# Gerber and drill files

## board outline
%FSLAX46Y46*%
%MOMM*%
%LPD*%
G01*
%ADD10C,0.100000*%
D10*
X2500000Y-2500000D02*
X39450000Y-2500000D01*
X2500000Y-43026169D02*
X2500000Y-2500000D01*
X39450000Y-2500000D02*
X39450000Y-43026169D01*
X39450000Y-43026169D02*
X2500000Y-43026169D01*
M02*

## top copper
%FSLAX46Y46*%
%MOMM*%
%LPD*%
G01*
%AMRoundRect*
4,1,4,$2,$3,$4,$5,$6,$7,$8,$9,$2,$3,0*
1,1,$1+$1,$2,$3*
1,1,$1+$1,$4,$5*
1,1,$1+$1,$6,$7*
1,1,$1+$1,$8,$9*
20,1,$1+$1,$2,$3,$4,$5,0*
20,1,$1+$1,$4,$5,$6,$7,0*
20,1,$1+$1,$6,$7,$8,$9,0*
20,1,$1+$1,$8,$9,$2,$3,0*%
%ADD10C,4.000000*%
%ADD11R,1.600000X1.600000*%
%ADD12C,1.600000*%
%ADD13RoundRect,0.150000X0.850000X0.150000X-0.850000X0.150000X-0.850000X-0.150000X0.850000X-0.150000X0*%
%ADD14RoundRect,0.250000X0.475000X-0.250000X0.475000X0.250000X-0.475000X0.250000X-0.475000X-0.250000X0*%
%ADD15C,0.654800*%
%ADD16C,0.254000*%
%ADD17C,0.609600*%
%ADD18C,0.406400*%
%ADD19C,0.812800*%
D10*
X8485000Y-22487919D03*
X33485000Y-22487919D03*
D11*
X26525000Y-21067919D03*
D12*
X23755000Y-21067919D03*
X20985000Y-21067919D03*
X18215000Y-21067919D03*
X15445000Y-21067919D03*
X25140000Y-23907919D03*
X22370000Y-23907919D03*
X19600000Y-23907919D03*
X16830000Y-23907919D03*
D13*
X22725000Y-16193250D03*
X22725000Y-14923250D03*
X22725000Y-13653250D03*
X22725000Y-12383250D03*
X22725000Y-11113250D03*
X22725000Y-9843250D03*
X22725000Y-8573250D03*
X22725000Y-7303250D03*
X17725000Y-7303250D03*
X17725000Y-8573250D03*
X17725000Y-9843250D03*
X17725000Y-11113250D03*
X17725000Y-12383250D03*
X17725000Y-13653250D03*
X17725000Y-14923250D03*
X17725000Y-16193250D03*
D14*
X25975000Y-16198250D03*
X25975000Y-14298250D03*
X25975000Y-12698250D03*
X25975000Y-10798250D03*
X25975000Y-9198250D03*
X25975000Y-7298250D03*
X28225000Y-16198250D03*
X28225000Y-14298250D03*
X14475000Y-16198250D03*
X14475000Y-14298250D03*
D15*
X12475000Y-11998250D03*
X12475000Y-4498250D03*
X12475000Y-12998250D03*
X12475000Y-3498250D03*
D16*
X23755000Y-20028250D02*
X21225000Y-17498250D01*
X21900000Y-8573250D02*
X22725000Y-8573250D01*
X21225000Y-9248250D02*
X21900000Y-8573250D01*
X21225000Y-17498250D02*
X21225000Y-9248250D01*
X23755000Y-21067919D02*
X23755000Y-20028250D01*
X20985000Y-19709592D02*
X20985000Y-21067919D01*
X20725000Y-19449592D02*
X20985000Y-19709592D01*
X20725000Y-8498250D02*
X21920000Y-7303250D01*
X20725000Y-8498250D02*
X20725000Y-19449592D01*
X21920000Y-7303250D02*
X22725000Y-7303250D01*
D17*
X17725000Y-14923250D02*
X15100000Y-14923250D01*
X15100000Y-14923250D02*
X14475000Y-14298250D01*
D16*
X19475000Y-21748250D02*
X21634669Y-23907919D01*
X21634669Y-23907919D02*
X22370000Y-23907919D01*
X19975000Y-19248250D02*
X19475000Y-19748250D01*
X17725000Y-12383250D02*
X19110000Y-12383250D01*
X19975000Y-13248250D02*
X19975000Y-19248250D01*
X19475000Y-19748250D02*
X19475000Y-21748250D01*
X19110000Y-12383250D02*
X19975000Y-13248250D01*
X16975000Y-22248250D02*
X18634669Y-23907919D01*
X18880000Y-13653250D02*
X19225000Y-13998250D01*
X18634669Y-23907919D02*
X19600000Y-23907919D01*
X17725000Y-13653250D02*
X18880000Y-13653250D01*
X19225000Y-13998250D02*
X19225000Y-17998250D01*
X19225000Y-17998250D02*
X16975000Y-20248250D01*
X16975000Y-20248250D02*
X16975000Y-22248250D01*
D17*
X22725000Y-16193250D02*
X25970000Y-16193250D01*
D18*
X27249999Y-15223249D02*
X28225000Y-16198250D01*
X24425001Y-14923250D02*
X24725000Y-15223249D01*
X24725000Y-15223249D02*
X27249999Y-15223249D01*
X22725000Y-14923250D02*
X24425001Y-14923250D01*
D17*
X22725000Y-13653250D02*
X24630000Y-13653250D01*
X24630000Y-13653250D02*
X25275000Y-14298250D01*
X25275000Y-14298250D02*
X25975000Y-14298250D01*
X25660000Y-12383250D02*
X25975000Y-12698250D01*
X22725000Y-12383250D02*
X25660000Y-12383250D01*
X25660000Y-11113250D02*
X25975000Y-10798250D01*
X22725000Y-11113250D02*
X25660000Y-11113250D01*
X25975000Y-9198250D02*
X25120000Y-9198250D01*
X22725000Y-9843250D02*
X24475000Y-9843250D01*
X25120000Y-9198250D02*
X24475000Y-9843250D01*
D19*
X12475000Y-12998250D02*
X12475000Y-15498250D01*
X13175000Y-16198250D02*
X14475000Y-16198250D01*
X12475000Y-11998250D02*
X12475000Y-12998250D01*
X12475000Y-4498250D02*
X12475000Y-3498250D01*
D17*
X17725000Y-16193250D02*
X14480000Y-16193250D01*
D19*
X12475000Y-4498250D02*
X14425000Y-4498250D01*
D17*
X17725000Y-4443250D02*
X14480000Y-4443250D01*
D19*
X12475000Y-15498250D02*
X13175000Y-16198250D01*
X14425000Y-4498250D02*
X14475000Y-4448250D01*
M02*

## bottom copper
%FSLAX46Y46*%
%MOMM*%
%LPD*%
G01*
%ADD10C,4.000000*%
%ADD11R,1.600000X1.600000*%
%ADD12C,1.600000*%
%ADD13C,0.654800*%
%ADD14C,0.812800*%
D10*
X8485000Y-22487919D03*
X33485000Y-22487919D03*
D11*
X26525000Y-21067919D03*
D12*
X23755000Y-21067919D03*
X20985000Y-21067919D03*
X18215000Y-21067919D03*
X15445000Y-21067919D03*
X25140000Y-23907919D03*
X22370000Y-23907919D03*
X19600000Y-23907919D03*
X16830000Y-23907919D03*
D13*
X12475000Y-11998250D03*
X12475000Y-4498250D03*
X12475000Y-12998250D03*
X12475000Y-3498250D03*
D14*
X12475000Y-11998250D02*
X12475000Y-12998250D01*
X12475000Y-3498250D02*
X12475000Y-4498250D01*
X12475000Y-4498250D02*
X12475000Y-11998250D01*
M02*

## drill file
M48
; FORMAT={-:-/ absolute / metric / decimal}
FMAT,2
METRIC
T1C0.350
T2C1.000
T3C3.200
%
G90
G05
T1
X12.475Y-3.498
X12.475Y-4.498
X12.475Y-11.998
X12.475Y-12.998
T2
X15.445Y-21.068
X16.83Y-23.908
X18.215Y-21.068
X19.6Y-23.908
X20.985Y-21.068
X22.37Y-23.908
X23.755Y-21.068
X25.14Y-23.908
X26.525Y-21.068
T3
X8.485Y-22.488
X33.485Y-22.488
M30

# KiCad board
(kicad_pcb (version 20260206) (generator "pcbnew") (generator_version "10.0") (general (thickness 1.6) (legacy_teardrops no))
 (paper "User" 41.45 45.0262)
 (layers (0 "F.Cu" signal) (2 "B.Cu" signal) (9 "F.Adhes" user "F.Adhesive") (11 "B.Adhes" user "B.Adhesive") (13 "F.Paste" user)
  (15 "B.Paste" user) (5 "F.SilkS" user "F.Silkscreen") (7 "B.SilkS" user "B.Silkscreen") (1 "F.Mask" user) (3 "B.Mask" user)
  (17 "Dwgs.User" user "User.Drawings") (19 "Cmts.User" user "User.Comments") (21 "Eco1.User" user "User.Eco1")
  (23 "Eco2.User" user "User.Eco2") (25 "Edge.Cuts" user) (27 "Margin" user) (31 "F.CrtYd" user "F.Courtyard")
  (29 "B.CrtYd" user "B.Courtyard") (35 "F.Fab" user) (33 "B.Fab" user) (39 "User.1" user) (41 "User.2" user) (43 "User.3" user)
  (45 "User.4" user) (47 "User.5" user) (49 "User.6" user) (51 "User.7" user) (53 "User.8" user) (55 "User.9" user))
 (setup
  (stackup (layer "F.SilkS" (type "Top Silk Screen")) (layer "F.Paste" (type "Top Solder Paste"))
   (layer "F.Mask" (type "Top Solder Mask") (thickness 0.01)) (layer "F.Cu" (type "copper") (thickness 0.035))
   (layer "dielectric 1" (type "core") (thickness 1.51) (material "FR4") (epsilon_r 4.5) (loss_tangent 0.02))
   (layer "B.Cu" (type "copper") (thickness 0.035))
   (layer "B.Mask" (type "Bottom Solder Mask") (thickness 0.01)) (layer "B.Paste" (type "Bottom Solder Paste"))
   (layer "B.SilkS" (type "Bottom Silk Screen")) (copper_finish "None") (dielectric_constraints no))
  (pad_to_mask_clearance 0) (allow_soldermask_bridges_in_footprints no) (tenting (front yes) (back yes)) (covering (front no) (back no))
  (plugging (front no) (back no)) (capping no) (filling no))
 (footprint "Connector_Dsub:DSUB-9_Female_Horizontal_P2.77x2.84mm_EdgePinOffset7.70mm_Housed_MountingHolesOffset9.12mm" (layer "F.Cu")
  (at 26.525 21.067919)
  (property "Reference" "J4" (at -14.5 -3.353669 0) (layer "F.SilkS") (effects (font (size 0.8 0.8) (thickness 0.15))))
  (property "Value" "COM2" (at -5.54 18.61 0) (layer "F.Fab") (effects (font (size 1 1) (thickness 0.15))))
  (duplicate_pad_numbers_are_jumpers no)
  (pad "0" thru_hole circle (at -18.04 1.42) (size 4 4) (drill 3.2) (layers "*.Cu" "*.Mask") (remove_unused_layers no)
   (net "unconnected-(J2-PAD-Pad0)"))
  (pad "0" thru_hole circle (at 6.96 1.42) (size 4 4) (drill 3.2) (layers "*.Cu" "*.Mask") (remove_unused_layers no)
   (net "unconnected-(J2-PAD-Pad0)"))
  (pad "1" thru_hole rect (at 0 0) (size 1.6 1.6) (drill 1) (layers "*.Cu" "*.Mask") (remove_unused_layers no) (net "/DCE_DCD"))
  (pad "2" thru_hole circle (at -2.77 0) (size 1.6 1.6) (drill 1) (layers "*.Cu" "*.Mask") (remove_unused_layers no) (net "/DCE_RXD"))
  (pad "3" thru_hole circle (at -5.54 0) (size 1.6 1.6) (drill 1) (layers "*.Cu" "*.Mask") (remove_unused_layers no) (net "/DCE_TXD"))
  (pad "4" thru_hole circle (at -8.31 0) (size 1.6 1.6) (drill 1) (layers "*.Cu" "*.Mask") (remove_unused_layers no) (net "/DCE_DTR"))
  (pad "5" thru_hole circle (at -11.08 0) (size 1.6 1.6) (drill 1) (layers "*.Cu" "*.Mask") (remove_unused_layers no) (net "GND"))
  (pad "6" thru_hole circle (at -1.385 2.84) (size 1.6 1.6) (drill 1) (layers "*.Cu" "*.Mask") (remove_unused_layers no) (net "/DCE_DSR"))
  (pad "7" thru_hole circle (at -4.155 2.84) (size 1.6 1.6) (drill 1) (layers "*.Cu" "*.Mask") (remove_unused_layers no) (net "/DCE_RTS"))
  (pad "8" thru_hole circle (at -6.925 2.84) (size 1.6 1.6) (drill 1) (layers "*.Cu" "*.Mask") (remove_unused_layers no) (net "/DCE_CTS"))
  (pad "9" thru_hole circle (at -9.695 2.84) (size 1.6 1.6) (drill 1) (layers "*.Cu" "*.Mask") (remove_unused_layers no) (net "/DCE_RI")))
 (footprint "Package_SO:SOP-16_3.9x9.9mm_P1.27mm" (layer "F.Cu") (at 20.225 11.74825 180)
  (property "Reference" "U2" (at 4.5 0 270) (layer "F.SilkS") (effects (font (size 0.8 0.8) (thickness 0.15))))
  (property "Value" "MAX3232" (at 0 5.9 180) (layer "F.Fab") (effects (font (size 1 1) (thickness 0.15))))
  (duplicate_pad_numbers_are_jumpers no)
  (pad "1" smd roundrect (at -2.5 -4.445 180) (size 2 0.6) (layers "F.Cu" "F.Mask" "F.Paste") (roundrect_rratio 0.25) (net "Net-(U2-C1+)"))
  (pad "2" smd roundrect (at -2.5 -3.175 180) (size 2 0.6) (layers "F.Cu" "F.Mask" "F.Paste") (roundrect_rratio 0.25) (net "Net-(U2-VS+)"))
  (pad "3" smd roundrect (at -2.5 -1.905 180) (size 2 0.6) (layers "F.Cu" "F.Mask" "F.Paste") (roundrect_rratio 0.25) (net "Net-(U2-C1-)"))
  (pad "4" smd roundrect (at -2.5 -0.635 180) (size 2 0.6) (layers "F.Cu" "F.Mask" "F.Paste") (roundrect_rratio 0.25) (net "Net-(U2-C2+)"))
  (pad "5" smd roundrect (at -2.5 0.635 180) (size 2 0.6) (layers "F.Cu" "F.Mask" "F.Paste") (roundrect_rratio 0.25) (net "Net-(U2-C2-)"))
  (pad "6" smd roundrect (at -2.5 1.905 180) (size 2 0.6) (layers "F.Cu" "F.Mask" "F.Paste") (roundrect_rratio 0.25) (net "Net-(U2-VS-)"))
  (pad "7" smd roundrect (at -2.5 3.175 180) (size 2 0.6) (layers "F.Cu" "F.Mask" "F.Paste") (roundrect_rratio 0.25) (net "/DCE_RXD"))
  (pad "8" smd roundrect (at -2.5 4.445 180) (size 2 0.6) (layers "F.Cu" "F.Mask" "F.Paste") (roundrect_rratio 0.25) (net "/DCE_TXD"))
  (pad "9" smd roundrect (at 2.5 4.445 180) (size 2 0.6) (layers "F.Cu" "F.Mask" "F.Paste") (roundrect_rratio 0.25) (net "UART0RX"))
  (pad "10" smd roundrect (at 2.5 3.175 180) (size 2 0.6) (layers "F.Cu" "F.Mask" "F.Paste") (roundrect_rratio 0.25) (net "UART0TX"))
  (pad "11" smd roundrect (at 2.5 1.905 180) (size 2 0.6) (layers "F.Cu" "F.Mask" "F.Paste") (roundrect_rratio 0.25) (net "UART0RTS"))
  (pad "12" smd roundrect (at 2.5 0.635 180) (size 2 0.6) (layers "F.Cu" "F.Mask" "F.Paste") (roundrect_rratio 0.25) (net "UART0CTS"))
  (pad "13" smd roundrect (at 2.5 -0.635 180) (size 2 0.6) (layers "F.Cu" "F.Mask" "F.Paste") (roundrect_rratio 0.25) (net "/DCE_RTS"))
  (pad "14" smd roundrect (at 2.5 -1.905 180) (size 2 0.6) (layers "F.Cu" "F.Mask" "F.Paste") (roundrect_rratio 0.25) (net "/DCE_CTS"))
  (pad "15" smd roundrect (at 2.5 -3.175 180) (size 2 0.6) (layers "F.Cu" "F.Mask" "F.Paste") (roundrect_rratio 0.25) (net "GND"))
  (pad "16" smd roundrect (at 2.5 -4.445 180) (size 2 0.6) (layers "F.Cu" "F.Mask" "F.Paste") (roundrect_rratio 0.25) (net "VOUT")))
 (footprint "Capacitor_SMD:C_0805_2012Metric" (layer "F.Cu") (at 25.975 15.24825 90)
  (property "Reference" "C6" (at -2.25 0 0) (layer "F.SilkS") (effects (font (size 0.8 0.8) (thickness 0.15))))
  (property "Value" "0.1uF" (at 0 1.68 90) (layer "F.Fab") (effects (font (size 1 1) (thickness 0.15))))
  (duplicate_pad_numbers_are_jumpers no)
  (pad "1" smd roundrect (at -0.95 0 90) (size 1 1.45) (layers "F.Cu" "F.Mask" "F.Paste") (roundrect_rratio 0.25) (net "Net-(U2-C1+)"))
  (pad "2" smd roundrect (at 0.95 0 90) (size 1 1.45) (layers "F.Cu" "F.Mask" "F.Paste") (roundrect_rratio 0.25) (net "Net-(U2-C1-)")))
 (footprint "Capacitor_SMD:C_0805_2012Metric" (layer "F.Cu") (at 25.975 11.74825 90)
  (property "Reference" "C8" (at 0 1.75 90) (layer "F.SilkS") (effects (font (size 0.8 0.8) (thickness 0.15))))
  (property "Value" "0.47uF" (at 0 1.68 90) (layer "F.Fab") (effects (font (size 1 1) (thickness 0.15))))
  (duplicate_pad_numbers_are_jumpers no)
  (pad "1" smd roundrect (at -0.95 0 90) (size 1 1.45) (layers "F.Cu" "F.Mask" "F.Paste") (roundrect_rratio 0.25) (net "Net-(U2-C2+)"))
  (pad "2" smd roundrect (at 0.95 0 90) (size 1 1.45) (layers "F.Cu" "F.Mask" "F.Paste") (roundrect_rratio 0.25) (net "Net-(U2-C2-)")))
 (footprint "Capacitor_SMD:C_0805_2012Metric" (layer "F.Cu") (at 25.975 8.24825 90)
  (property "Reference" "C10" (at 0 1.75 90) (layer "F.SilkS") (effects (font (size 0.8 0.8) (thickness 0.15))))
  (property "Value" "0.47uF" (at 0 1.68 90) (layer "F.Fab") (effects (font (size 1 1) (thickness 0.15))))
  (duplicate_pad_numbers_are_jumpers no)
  (pad "1" smd roundrect (at -0.95 0 90) (size 1 1.45) (layers "F.Cu" "F.Mask" "F.Paste") (roundrect_rratio 0.25) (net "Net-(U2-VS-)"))
  (pad "2" smd roundrect (at 0.95 0 90) (size 1 1.45) (layers "F.Cu" "F.Mask" "F.Paste") (roundrect_rratio 0.25) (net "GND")))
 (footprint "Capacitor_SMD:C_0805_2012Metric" (layer "F.Cu") (at 28.225 15.24825 90)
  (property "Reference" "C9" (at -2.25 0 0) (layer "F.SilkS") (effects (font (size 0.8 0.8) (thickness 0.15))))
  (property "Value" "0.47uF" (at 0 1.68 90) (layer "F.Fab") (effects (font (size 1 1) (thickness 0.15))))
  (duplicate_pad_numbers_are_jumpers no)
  (pad "1" smd roundrect (at -0.95 0 90) (size 1 1.45) (layers "F.Cu" "F.Mask" "F.Paste") (roundrect_rratio 0.25) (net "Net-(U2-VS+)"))
  (pad "2" smd roundrect (at 0.95 0 90) (size 1 1.45) (layers "F.Cu" "F.Mask" "F.Paste") (roundrect_rratio 0.25) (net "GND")))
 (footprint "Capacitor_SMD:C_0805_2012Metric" (layer "F.Cu") (at 14.475 15.24825 90)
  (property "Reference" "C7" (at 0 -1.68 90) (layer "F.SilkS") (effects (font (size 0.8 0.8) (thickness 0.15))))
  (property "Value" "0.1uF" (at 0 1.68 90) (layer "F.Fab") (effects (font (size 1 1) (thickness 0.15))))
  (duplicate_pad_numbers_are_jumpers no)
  (pad "1" smd roundrect (at -0.95 0 90) (size 1 1.45) (layers "F.Cu" "F.Mask" "F.Paste") (roundrect_rratio 0.25) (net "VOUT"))
  (pad "2" smd roundrect (at 0.95 0 90) (size 1 1.45) (layers "F.Cu" "F.Mask" "F.Paste") (roundrect_rratio 0.25) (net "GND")))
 (gr_line (start 2.5 2.5) (end 39.45 2.5) (stroke (width 0.1) (type default)) (layer "Edge.Cuts"))
 (gr_line (start 2.5 43.026169) (end 2.5 2.5) (stroke (width 0.1) (type default)) (layer "Edge.Cuts"))
 (gr_line (start 39.45 2.5) (end 39.45 43.026169) (stroke (width 0.1) (type default)) (layer "Edge.Cuts"))
 (gr_line (start 39.45 43.026169) (end 2.5 43.026169) (stroke (width 0.1) (type default)) (layer "Edge.Cuts"))
 (segment (start 23.755 20.02825) (end 21.225 17.49825) (width 0.254) (layer "F.Cu") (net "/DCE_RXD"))
 (segment (start 21.9 8.57325) (end 22.725 8.57325) (width 0.254) (layer "F.Cu") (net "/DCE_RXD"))
 (segment (start 21.225 9.24825) (end 21.9 8.57325) (width 0.254) (layer "F.Cu") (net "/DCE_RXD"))
 (segment (start 21.225 17.49825) (end 21.225 9.24825) (width 0.254) (layer "F.Cu") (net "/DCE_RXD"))
 (segment (start 23.755 21.067919) (end 23.755 20.02825) (width 0.254) (layer "F.Cu") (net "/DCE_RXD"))
 (segment (start 20.985 19.709592) (end 20.985 21.067919) (width 0.254) (layer "F.Cu") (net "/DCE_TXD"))
 (segment (start 20.725 19.449592) (end 20.985 19.709592) (width 0.254) (layer "F.Cu") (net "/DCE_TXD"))
 (segment (start 20.725 8.49825) (end 21.92 7.30325) (width 0.254) (layer "F.Cu") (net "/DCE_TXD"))
 (segment (start 20.725 8.49825) (end 20.725 19.449592) (width 0.254) (layer "F.Cu") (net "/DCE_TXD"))
 (segment (start 21.92 7.30325) (end 22.725 7.30325) (width 0.254) (layer "F.Cu") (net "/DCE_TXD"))
 (segment (start 17.725 14.92325) (end 15.1 14.92325) (width 0.6096) (layer "F.Cu") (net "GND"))
 (segment (start 15.1 14.92325) (end 14.475 14.29825) (width 0.6096) (layer "F.Cu") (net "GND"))
 (segment (start 19.475 21.74825) (end 21.634669 23.907919) (width 0.254) (layer "F.Cu") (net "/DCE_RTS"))
 (segment (start 21.634669 23.907919) (end 22.37 23.907919) (width 0.254) (layer "F.Cu") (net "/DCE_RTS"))
 (segment (start 19.975 19.24825) (end 19.475 19.74825) (width 0.254) (layer "F.Cu") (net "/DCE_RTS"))
 (segment (start 17.725 12.38325) (end 19.11 12.38325) (width 0.254) (layer "F.Cu") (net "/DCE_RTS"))
 (segment (start 19.975 13.24825) (end 19.975 19.24825) (width 0.254) (layer "F.Cu") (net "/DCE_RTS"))
 (segment (start 19.475 19.74825) (end 19.475 21.74825) (width 0.254) (layer "F.Cu") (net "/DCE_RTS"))
 (segment (start 19.11 12.38325) (end 19.975 13.24825) (width 0.254) (layer "F.Cu") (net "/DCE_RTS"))
 (segment (start 16.975 22.24825) (end 18.634669 23.907919) (width 0.254) (layer "F.Cu") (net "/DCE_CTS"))
 (segment (start 18.88 13.65325) (end 19.225 13.99825) (width 0.254) (layer "F.Cu") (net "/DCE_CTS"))
 (segment (start 18.634669 23.907919) (end 19.6 23.907919) (width 0.254) (layer "F.Cu") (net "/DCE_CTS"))
 (segment (start 17.725 13.65325) (end 18.88 13.65325) (width 0.254) (layer "F.Cu") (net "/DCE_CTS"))
 (segment (start 19.225 13.99825) (end 19.225 17.99825) (width 0.254) (layer "F.Cu") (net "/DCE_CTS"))
 (segment (start 19.225 17.99825) (end 16.975 20.24825) (width 0.254) (layer "F.Cu") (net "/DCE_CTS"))
 (segment (start 16.975 20.24825) (end 16.975 22.24825) (width 0.254) (layer "F.Cu") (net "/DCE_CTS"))
 (segment (start 22.725 16.19325) (end 25.97 16.19325) (width 0.6096) (layer "F.Cu") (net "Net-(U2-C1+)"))
 (segment (start 27.249999 15.223249) (end 28.225 16.19825) (width 0.4064) (layer "F.Cu") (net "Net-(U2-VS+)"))
 (segment (start 24.425001 14.92325) (end 24.725 15.223249) (width 0.4064) (layer "F.Cu") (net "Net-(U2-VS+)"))
 (segment (start 24.725 15.223249) (end 27.249999 15.223249) (width 0.4064) (layer "F.Cu") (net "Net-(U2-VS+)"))
 (segment (start 22.725 14.92325) (end 24.425001 14.92325) (width 0.4064) (layer "F.Cu") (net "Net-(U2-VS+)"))
 (segment (start 22.725 13.65325) (end 24.63 13.65325) (width 0.6096) (layer "F.Cu") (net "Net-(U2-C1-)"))
 (segment (start 24.63 13.65325) (end 25.275 14.29825) (width 0.6096) (layer "F.Cu") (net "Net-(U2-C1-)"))
 (segment (start 25.275 14.29825) (end 25.975 14.29825) (width 0.6096) (layer "F.Cu") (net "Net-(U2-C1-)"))
 (segment (start 25.66 12.38325) (end 25.975 12.69825) (width 0.6096) (layer "F.Cu") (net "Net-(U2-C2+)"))
 (segment (start 22.725 12.38325) (end 25.66 12.38325) (width 0.6096) (layer "F.Cu") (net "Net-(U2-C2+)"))
 (segment (start 25.66 11.11325) (end 25.975 10.79825) (width 0.6096) (layer "F.Cu") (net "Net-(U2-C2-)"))
 (segment (start 22.725 11.11325) (end 25.66 11.11325) (width 0.6096) (layer "F.Cu") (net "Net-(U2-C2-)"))
 (segment (start 25.975 9.19825) (end 25.12 9.19825) (width 0.6096) (layer "F.Cu") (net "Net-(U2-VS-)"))
 (segment (start 22.725 9.84325) (end 24.475 9.84325) (width 0.6096) (layer "F.Cu") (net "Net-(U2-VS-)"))
 (segment (start 25.12 9.19825) (end 24.475 9.84325) (width 0.6096) (layer "F.Cu") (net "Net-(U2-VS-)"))
 (segment (start 12.475 12.99825) (end 12.475 15.49825) (width 0.8128) (layer "F.Cu") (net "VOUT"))
 (segment (start 13.175 16.19825) (end 14.475 16.19825) (width 0.8128) (layer "F.Cu") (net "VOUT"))
 (segment (start 12.475 11.99825) (end 12.475 12.99825) (width 0.8128) (layer "F.Cu") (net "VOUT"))
 (segment (start 12.475 4.49825) (end 12.475 3.49825) (width 0.8128) (layer "F.Cu") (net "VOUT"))
 (segment (start 17.725 16.19325) (end 14.48 16.19325) (width 0.6096) (layer "F.Cu") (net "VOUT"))
 (segment (start 12.475 4.49825) (end 14.425 4.49825) (width 0.8128) (layer "F.Cu") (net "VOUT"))
 (segment (start 17.725 4.44325) (end 14.48 4.44325) (width 0.6096) (layer "F.Cu") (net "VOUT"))
 (segment (start 12.475 15.49825) (end 13.175 16.19825) (width 0.8128) (layer "F.Cu") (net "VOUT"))
 (segment (start 14.425 4.49825) (end 14.475 4.44825) (width 0.8128) (layer "F.Cu") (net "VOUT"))
 (via (at 12.475 11.99825) (size 0.6548) (drill 0.35) (layers "F.Cu" "B.Cu") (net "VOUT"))
 (via (at 12.475 4.49825) (size 0.6548) (drill 0.35) (layers "F.Cu" "B.Cu") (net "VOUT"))
 (via (at 12.475 12.99825) (size 0.6548) (drill 0.35) (layers "F.Cu" "B.Cu") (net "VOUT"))
 (via (at 12.475 3.49825) (size 0.6548) (drill 0.35) (layers "F.Cu" "B.Cu") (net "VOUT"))
 (segment (start 12.475 11.99825) (end 12.475 12.99825) (width 0.8128) (layer "B.Cu") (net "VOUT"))
 (segment (start 12.475 3.49825) (end 12.475 4.49825) (width 0.8128) (layer "B.Cu") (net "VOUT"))
 (segment (start 12.475 4.49825) (end 12.475 11.99825) (width 0.8128) (layer "B.Cu") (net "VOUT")))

